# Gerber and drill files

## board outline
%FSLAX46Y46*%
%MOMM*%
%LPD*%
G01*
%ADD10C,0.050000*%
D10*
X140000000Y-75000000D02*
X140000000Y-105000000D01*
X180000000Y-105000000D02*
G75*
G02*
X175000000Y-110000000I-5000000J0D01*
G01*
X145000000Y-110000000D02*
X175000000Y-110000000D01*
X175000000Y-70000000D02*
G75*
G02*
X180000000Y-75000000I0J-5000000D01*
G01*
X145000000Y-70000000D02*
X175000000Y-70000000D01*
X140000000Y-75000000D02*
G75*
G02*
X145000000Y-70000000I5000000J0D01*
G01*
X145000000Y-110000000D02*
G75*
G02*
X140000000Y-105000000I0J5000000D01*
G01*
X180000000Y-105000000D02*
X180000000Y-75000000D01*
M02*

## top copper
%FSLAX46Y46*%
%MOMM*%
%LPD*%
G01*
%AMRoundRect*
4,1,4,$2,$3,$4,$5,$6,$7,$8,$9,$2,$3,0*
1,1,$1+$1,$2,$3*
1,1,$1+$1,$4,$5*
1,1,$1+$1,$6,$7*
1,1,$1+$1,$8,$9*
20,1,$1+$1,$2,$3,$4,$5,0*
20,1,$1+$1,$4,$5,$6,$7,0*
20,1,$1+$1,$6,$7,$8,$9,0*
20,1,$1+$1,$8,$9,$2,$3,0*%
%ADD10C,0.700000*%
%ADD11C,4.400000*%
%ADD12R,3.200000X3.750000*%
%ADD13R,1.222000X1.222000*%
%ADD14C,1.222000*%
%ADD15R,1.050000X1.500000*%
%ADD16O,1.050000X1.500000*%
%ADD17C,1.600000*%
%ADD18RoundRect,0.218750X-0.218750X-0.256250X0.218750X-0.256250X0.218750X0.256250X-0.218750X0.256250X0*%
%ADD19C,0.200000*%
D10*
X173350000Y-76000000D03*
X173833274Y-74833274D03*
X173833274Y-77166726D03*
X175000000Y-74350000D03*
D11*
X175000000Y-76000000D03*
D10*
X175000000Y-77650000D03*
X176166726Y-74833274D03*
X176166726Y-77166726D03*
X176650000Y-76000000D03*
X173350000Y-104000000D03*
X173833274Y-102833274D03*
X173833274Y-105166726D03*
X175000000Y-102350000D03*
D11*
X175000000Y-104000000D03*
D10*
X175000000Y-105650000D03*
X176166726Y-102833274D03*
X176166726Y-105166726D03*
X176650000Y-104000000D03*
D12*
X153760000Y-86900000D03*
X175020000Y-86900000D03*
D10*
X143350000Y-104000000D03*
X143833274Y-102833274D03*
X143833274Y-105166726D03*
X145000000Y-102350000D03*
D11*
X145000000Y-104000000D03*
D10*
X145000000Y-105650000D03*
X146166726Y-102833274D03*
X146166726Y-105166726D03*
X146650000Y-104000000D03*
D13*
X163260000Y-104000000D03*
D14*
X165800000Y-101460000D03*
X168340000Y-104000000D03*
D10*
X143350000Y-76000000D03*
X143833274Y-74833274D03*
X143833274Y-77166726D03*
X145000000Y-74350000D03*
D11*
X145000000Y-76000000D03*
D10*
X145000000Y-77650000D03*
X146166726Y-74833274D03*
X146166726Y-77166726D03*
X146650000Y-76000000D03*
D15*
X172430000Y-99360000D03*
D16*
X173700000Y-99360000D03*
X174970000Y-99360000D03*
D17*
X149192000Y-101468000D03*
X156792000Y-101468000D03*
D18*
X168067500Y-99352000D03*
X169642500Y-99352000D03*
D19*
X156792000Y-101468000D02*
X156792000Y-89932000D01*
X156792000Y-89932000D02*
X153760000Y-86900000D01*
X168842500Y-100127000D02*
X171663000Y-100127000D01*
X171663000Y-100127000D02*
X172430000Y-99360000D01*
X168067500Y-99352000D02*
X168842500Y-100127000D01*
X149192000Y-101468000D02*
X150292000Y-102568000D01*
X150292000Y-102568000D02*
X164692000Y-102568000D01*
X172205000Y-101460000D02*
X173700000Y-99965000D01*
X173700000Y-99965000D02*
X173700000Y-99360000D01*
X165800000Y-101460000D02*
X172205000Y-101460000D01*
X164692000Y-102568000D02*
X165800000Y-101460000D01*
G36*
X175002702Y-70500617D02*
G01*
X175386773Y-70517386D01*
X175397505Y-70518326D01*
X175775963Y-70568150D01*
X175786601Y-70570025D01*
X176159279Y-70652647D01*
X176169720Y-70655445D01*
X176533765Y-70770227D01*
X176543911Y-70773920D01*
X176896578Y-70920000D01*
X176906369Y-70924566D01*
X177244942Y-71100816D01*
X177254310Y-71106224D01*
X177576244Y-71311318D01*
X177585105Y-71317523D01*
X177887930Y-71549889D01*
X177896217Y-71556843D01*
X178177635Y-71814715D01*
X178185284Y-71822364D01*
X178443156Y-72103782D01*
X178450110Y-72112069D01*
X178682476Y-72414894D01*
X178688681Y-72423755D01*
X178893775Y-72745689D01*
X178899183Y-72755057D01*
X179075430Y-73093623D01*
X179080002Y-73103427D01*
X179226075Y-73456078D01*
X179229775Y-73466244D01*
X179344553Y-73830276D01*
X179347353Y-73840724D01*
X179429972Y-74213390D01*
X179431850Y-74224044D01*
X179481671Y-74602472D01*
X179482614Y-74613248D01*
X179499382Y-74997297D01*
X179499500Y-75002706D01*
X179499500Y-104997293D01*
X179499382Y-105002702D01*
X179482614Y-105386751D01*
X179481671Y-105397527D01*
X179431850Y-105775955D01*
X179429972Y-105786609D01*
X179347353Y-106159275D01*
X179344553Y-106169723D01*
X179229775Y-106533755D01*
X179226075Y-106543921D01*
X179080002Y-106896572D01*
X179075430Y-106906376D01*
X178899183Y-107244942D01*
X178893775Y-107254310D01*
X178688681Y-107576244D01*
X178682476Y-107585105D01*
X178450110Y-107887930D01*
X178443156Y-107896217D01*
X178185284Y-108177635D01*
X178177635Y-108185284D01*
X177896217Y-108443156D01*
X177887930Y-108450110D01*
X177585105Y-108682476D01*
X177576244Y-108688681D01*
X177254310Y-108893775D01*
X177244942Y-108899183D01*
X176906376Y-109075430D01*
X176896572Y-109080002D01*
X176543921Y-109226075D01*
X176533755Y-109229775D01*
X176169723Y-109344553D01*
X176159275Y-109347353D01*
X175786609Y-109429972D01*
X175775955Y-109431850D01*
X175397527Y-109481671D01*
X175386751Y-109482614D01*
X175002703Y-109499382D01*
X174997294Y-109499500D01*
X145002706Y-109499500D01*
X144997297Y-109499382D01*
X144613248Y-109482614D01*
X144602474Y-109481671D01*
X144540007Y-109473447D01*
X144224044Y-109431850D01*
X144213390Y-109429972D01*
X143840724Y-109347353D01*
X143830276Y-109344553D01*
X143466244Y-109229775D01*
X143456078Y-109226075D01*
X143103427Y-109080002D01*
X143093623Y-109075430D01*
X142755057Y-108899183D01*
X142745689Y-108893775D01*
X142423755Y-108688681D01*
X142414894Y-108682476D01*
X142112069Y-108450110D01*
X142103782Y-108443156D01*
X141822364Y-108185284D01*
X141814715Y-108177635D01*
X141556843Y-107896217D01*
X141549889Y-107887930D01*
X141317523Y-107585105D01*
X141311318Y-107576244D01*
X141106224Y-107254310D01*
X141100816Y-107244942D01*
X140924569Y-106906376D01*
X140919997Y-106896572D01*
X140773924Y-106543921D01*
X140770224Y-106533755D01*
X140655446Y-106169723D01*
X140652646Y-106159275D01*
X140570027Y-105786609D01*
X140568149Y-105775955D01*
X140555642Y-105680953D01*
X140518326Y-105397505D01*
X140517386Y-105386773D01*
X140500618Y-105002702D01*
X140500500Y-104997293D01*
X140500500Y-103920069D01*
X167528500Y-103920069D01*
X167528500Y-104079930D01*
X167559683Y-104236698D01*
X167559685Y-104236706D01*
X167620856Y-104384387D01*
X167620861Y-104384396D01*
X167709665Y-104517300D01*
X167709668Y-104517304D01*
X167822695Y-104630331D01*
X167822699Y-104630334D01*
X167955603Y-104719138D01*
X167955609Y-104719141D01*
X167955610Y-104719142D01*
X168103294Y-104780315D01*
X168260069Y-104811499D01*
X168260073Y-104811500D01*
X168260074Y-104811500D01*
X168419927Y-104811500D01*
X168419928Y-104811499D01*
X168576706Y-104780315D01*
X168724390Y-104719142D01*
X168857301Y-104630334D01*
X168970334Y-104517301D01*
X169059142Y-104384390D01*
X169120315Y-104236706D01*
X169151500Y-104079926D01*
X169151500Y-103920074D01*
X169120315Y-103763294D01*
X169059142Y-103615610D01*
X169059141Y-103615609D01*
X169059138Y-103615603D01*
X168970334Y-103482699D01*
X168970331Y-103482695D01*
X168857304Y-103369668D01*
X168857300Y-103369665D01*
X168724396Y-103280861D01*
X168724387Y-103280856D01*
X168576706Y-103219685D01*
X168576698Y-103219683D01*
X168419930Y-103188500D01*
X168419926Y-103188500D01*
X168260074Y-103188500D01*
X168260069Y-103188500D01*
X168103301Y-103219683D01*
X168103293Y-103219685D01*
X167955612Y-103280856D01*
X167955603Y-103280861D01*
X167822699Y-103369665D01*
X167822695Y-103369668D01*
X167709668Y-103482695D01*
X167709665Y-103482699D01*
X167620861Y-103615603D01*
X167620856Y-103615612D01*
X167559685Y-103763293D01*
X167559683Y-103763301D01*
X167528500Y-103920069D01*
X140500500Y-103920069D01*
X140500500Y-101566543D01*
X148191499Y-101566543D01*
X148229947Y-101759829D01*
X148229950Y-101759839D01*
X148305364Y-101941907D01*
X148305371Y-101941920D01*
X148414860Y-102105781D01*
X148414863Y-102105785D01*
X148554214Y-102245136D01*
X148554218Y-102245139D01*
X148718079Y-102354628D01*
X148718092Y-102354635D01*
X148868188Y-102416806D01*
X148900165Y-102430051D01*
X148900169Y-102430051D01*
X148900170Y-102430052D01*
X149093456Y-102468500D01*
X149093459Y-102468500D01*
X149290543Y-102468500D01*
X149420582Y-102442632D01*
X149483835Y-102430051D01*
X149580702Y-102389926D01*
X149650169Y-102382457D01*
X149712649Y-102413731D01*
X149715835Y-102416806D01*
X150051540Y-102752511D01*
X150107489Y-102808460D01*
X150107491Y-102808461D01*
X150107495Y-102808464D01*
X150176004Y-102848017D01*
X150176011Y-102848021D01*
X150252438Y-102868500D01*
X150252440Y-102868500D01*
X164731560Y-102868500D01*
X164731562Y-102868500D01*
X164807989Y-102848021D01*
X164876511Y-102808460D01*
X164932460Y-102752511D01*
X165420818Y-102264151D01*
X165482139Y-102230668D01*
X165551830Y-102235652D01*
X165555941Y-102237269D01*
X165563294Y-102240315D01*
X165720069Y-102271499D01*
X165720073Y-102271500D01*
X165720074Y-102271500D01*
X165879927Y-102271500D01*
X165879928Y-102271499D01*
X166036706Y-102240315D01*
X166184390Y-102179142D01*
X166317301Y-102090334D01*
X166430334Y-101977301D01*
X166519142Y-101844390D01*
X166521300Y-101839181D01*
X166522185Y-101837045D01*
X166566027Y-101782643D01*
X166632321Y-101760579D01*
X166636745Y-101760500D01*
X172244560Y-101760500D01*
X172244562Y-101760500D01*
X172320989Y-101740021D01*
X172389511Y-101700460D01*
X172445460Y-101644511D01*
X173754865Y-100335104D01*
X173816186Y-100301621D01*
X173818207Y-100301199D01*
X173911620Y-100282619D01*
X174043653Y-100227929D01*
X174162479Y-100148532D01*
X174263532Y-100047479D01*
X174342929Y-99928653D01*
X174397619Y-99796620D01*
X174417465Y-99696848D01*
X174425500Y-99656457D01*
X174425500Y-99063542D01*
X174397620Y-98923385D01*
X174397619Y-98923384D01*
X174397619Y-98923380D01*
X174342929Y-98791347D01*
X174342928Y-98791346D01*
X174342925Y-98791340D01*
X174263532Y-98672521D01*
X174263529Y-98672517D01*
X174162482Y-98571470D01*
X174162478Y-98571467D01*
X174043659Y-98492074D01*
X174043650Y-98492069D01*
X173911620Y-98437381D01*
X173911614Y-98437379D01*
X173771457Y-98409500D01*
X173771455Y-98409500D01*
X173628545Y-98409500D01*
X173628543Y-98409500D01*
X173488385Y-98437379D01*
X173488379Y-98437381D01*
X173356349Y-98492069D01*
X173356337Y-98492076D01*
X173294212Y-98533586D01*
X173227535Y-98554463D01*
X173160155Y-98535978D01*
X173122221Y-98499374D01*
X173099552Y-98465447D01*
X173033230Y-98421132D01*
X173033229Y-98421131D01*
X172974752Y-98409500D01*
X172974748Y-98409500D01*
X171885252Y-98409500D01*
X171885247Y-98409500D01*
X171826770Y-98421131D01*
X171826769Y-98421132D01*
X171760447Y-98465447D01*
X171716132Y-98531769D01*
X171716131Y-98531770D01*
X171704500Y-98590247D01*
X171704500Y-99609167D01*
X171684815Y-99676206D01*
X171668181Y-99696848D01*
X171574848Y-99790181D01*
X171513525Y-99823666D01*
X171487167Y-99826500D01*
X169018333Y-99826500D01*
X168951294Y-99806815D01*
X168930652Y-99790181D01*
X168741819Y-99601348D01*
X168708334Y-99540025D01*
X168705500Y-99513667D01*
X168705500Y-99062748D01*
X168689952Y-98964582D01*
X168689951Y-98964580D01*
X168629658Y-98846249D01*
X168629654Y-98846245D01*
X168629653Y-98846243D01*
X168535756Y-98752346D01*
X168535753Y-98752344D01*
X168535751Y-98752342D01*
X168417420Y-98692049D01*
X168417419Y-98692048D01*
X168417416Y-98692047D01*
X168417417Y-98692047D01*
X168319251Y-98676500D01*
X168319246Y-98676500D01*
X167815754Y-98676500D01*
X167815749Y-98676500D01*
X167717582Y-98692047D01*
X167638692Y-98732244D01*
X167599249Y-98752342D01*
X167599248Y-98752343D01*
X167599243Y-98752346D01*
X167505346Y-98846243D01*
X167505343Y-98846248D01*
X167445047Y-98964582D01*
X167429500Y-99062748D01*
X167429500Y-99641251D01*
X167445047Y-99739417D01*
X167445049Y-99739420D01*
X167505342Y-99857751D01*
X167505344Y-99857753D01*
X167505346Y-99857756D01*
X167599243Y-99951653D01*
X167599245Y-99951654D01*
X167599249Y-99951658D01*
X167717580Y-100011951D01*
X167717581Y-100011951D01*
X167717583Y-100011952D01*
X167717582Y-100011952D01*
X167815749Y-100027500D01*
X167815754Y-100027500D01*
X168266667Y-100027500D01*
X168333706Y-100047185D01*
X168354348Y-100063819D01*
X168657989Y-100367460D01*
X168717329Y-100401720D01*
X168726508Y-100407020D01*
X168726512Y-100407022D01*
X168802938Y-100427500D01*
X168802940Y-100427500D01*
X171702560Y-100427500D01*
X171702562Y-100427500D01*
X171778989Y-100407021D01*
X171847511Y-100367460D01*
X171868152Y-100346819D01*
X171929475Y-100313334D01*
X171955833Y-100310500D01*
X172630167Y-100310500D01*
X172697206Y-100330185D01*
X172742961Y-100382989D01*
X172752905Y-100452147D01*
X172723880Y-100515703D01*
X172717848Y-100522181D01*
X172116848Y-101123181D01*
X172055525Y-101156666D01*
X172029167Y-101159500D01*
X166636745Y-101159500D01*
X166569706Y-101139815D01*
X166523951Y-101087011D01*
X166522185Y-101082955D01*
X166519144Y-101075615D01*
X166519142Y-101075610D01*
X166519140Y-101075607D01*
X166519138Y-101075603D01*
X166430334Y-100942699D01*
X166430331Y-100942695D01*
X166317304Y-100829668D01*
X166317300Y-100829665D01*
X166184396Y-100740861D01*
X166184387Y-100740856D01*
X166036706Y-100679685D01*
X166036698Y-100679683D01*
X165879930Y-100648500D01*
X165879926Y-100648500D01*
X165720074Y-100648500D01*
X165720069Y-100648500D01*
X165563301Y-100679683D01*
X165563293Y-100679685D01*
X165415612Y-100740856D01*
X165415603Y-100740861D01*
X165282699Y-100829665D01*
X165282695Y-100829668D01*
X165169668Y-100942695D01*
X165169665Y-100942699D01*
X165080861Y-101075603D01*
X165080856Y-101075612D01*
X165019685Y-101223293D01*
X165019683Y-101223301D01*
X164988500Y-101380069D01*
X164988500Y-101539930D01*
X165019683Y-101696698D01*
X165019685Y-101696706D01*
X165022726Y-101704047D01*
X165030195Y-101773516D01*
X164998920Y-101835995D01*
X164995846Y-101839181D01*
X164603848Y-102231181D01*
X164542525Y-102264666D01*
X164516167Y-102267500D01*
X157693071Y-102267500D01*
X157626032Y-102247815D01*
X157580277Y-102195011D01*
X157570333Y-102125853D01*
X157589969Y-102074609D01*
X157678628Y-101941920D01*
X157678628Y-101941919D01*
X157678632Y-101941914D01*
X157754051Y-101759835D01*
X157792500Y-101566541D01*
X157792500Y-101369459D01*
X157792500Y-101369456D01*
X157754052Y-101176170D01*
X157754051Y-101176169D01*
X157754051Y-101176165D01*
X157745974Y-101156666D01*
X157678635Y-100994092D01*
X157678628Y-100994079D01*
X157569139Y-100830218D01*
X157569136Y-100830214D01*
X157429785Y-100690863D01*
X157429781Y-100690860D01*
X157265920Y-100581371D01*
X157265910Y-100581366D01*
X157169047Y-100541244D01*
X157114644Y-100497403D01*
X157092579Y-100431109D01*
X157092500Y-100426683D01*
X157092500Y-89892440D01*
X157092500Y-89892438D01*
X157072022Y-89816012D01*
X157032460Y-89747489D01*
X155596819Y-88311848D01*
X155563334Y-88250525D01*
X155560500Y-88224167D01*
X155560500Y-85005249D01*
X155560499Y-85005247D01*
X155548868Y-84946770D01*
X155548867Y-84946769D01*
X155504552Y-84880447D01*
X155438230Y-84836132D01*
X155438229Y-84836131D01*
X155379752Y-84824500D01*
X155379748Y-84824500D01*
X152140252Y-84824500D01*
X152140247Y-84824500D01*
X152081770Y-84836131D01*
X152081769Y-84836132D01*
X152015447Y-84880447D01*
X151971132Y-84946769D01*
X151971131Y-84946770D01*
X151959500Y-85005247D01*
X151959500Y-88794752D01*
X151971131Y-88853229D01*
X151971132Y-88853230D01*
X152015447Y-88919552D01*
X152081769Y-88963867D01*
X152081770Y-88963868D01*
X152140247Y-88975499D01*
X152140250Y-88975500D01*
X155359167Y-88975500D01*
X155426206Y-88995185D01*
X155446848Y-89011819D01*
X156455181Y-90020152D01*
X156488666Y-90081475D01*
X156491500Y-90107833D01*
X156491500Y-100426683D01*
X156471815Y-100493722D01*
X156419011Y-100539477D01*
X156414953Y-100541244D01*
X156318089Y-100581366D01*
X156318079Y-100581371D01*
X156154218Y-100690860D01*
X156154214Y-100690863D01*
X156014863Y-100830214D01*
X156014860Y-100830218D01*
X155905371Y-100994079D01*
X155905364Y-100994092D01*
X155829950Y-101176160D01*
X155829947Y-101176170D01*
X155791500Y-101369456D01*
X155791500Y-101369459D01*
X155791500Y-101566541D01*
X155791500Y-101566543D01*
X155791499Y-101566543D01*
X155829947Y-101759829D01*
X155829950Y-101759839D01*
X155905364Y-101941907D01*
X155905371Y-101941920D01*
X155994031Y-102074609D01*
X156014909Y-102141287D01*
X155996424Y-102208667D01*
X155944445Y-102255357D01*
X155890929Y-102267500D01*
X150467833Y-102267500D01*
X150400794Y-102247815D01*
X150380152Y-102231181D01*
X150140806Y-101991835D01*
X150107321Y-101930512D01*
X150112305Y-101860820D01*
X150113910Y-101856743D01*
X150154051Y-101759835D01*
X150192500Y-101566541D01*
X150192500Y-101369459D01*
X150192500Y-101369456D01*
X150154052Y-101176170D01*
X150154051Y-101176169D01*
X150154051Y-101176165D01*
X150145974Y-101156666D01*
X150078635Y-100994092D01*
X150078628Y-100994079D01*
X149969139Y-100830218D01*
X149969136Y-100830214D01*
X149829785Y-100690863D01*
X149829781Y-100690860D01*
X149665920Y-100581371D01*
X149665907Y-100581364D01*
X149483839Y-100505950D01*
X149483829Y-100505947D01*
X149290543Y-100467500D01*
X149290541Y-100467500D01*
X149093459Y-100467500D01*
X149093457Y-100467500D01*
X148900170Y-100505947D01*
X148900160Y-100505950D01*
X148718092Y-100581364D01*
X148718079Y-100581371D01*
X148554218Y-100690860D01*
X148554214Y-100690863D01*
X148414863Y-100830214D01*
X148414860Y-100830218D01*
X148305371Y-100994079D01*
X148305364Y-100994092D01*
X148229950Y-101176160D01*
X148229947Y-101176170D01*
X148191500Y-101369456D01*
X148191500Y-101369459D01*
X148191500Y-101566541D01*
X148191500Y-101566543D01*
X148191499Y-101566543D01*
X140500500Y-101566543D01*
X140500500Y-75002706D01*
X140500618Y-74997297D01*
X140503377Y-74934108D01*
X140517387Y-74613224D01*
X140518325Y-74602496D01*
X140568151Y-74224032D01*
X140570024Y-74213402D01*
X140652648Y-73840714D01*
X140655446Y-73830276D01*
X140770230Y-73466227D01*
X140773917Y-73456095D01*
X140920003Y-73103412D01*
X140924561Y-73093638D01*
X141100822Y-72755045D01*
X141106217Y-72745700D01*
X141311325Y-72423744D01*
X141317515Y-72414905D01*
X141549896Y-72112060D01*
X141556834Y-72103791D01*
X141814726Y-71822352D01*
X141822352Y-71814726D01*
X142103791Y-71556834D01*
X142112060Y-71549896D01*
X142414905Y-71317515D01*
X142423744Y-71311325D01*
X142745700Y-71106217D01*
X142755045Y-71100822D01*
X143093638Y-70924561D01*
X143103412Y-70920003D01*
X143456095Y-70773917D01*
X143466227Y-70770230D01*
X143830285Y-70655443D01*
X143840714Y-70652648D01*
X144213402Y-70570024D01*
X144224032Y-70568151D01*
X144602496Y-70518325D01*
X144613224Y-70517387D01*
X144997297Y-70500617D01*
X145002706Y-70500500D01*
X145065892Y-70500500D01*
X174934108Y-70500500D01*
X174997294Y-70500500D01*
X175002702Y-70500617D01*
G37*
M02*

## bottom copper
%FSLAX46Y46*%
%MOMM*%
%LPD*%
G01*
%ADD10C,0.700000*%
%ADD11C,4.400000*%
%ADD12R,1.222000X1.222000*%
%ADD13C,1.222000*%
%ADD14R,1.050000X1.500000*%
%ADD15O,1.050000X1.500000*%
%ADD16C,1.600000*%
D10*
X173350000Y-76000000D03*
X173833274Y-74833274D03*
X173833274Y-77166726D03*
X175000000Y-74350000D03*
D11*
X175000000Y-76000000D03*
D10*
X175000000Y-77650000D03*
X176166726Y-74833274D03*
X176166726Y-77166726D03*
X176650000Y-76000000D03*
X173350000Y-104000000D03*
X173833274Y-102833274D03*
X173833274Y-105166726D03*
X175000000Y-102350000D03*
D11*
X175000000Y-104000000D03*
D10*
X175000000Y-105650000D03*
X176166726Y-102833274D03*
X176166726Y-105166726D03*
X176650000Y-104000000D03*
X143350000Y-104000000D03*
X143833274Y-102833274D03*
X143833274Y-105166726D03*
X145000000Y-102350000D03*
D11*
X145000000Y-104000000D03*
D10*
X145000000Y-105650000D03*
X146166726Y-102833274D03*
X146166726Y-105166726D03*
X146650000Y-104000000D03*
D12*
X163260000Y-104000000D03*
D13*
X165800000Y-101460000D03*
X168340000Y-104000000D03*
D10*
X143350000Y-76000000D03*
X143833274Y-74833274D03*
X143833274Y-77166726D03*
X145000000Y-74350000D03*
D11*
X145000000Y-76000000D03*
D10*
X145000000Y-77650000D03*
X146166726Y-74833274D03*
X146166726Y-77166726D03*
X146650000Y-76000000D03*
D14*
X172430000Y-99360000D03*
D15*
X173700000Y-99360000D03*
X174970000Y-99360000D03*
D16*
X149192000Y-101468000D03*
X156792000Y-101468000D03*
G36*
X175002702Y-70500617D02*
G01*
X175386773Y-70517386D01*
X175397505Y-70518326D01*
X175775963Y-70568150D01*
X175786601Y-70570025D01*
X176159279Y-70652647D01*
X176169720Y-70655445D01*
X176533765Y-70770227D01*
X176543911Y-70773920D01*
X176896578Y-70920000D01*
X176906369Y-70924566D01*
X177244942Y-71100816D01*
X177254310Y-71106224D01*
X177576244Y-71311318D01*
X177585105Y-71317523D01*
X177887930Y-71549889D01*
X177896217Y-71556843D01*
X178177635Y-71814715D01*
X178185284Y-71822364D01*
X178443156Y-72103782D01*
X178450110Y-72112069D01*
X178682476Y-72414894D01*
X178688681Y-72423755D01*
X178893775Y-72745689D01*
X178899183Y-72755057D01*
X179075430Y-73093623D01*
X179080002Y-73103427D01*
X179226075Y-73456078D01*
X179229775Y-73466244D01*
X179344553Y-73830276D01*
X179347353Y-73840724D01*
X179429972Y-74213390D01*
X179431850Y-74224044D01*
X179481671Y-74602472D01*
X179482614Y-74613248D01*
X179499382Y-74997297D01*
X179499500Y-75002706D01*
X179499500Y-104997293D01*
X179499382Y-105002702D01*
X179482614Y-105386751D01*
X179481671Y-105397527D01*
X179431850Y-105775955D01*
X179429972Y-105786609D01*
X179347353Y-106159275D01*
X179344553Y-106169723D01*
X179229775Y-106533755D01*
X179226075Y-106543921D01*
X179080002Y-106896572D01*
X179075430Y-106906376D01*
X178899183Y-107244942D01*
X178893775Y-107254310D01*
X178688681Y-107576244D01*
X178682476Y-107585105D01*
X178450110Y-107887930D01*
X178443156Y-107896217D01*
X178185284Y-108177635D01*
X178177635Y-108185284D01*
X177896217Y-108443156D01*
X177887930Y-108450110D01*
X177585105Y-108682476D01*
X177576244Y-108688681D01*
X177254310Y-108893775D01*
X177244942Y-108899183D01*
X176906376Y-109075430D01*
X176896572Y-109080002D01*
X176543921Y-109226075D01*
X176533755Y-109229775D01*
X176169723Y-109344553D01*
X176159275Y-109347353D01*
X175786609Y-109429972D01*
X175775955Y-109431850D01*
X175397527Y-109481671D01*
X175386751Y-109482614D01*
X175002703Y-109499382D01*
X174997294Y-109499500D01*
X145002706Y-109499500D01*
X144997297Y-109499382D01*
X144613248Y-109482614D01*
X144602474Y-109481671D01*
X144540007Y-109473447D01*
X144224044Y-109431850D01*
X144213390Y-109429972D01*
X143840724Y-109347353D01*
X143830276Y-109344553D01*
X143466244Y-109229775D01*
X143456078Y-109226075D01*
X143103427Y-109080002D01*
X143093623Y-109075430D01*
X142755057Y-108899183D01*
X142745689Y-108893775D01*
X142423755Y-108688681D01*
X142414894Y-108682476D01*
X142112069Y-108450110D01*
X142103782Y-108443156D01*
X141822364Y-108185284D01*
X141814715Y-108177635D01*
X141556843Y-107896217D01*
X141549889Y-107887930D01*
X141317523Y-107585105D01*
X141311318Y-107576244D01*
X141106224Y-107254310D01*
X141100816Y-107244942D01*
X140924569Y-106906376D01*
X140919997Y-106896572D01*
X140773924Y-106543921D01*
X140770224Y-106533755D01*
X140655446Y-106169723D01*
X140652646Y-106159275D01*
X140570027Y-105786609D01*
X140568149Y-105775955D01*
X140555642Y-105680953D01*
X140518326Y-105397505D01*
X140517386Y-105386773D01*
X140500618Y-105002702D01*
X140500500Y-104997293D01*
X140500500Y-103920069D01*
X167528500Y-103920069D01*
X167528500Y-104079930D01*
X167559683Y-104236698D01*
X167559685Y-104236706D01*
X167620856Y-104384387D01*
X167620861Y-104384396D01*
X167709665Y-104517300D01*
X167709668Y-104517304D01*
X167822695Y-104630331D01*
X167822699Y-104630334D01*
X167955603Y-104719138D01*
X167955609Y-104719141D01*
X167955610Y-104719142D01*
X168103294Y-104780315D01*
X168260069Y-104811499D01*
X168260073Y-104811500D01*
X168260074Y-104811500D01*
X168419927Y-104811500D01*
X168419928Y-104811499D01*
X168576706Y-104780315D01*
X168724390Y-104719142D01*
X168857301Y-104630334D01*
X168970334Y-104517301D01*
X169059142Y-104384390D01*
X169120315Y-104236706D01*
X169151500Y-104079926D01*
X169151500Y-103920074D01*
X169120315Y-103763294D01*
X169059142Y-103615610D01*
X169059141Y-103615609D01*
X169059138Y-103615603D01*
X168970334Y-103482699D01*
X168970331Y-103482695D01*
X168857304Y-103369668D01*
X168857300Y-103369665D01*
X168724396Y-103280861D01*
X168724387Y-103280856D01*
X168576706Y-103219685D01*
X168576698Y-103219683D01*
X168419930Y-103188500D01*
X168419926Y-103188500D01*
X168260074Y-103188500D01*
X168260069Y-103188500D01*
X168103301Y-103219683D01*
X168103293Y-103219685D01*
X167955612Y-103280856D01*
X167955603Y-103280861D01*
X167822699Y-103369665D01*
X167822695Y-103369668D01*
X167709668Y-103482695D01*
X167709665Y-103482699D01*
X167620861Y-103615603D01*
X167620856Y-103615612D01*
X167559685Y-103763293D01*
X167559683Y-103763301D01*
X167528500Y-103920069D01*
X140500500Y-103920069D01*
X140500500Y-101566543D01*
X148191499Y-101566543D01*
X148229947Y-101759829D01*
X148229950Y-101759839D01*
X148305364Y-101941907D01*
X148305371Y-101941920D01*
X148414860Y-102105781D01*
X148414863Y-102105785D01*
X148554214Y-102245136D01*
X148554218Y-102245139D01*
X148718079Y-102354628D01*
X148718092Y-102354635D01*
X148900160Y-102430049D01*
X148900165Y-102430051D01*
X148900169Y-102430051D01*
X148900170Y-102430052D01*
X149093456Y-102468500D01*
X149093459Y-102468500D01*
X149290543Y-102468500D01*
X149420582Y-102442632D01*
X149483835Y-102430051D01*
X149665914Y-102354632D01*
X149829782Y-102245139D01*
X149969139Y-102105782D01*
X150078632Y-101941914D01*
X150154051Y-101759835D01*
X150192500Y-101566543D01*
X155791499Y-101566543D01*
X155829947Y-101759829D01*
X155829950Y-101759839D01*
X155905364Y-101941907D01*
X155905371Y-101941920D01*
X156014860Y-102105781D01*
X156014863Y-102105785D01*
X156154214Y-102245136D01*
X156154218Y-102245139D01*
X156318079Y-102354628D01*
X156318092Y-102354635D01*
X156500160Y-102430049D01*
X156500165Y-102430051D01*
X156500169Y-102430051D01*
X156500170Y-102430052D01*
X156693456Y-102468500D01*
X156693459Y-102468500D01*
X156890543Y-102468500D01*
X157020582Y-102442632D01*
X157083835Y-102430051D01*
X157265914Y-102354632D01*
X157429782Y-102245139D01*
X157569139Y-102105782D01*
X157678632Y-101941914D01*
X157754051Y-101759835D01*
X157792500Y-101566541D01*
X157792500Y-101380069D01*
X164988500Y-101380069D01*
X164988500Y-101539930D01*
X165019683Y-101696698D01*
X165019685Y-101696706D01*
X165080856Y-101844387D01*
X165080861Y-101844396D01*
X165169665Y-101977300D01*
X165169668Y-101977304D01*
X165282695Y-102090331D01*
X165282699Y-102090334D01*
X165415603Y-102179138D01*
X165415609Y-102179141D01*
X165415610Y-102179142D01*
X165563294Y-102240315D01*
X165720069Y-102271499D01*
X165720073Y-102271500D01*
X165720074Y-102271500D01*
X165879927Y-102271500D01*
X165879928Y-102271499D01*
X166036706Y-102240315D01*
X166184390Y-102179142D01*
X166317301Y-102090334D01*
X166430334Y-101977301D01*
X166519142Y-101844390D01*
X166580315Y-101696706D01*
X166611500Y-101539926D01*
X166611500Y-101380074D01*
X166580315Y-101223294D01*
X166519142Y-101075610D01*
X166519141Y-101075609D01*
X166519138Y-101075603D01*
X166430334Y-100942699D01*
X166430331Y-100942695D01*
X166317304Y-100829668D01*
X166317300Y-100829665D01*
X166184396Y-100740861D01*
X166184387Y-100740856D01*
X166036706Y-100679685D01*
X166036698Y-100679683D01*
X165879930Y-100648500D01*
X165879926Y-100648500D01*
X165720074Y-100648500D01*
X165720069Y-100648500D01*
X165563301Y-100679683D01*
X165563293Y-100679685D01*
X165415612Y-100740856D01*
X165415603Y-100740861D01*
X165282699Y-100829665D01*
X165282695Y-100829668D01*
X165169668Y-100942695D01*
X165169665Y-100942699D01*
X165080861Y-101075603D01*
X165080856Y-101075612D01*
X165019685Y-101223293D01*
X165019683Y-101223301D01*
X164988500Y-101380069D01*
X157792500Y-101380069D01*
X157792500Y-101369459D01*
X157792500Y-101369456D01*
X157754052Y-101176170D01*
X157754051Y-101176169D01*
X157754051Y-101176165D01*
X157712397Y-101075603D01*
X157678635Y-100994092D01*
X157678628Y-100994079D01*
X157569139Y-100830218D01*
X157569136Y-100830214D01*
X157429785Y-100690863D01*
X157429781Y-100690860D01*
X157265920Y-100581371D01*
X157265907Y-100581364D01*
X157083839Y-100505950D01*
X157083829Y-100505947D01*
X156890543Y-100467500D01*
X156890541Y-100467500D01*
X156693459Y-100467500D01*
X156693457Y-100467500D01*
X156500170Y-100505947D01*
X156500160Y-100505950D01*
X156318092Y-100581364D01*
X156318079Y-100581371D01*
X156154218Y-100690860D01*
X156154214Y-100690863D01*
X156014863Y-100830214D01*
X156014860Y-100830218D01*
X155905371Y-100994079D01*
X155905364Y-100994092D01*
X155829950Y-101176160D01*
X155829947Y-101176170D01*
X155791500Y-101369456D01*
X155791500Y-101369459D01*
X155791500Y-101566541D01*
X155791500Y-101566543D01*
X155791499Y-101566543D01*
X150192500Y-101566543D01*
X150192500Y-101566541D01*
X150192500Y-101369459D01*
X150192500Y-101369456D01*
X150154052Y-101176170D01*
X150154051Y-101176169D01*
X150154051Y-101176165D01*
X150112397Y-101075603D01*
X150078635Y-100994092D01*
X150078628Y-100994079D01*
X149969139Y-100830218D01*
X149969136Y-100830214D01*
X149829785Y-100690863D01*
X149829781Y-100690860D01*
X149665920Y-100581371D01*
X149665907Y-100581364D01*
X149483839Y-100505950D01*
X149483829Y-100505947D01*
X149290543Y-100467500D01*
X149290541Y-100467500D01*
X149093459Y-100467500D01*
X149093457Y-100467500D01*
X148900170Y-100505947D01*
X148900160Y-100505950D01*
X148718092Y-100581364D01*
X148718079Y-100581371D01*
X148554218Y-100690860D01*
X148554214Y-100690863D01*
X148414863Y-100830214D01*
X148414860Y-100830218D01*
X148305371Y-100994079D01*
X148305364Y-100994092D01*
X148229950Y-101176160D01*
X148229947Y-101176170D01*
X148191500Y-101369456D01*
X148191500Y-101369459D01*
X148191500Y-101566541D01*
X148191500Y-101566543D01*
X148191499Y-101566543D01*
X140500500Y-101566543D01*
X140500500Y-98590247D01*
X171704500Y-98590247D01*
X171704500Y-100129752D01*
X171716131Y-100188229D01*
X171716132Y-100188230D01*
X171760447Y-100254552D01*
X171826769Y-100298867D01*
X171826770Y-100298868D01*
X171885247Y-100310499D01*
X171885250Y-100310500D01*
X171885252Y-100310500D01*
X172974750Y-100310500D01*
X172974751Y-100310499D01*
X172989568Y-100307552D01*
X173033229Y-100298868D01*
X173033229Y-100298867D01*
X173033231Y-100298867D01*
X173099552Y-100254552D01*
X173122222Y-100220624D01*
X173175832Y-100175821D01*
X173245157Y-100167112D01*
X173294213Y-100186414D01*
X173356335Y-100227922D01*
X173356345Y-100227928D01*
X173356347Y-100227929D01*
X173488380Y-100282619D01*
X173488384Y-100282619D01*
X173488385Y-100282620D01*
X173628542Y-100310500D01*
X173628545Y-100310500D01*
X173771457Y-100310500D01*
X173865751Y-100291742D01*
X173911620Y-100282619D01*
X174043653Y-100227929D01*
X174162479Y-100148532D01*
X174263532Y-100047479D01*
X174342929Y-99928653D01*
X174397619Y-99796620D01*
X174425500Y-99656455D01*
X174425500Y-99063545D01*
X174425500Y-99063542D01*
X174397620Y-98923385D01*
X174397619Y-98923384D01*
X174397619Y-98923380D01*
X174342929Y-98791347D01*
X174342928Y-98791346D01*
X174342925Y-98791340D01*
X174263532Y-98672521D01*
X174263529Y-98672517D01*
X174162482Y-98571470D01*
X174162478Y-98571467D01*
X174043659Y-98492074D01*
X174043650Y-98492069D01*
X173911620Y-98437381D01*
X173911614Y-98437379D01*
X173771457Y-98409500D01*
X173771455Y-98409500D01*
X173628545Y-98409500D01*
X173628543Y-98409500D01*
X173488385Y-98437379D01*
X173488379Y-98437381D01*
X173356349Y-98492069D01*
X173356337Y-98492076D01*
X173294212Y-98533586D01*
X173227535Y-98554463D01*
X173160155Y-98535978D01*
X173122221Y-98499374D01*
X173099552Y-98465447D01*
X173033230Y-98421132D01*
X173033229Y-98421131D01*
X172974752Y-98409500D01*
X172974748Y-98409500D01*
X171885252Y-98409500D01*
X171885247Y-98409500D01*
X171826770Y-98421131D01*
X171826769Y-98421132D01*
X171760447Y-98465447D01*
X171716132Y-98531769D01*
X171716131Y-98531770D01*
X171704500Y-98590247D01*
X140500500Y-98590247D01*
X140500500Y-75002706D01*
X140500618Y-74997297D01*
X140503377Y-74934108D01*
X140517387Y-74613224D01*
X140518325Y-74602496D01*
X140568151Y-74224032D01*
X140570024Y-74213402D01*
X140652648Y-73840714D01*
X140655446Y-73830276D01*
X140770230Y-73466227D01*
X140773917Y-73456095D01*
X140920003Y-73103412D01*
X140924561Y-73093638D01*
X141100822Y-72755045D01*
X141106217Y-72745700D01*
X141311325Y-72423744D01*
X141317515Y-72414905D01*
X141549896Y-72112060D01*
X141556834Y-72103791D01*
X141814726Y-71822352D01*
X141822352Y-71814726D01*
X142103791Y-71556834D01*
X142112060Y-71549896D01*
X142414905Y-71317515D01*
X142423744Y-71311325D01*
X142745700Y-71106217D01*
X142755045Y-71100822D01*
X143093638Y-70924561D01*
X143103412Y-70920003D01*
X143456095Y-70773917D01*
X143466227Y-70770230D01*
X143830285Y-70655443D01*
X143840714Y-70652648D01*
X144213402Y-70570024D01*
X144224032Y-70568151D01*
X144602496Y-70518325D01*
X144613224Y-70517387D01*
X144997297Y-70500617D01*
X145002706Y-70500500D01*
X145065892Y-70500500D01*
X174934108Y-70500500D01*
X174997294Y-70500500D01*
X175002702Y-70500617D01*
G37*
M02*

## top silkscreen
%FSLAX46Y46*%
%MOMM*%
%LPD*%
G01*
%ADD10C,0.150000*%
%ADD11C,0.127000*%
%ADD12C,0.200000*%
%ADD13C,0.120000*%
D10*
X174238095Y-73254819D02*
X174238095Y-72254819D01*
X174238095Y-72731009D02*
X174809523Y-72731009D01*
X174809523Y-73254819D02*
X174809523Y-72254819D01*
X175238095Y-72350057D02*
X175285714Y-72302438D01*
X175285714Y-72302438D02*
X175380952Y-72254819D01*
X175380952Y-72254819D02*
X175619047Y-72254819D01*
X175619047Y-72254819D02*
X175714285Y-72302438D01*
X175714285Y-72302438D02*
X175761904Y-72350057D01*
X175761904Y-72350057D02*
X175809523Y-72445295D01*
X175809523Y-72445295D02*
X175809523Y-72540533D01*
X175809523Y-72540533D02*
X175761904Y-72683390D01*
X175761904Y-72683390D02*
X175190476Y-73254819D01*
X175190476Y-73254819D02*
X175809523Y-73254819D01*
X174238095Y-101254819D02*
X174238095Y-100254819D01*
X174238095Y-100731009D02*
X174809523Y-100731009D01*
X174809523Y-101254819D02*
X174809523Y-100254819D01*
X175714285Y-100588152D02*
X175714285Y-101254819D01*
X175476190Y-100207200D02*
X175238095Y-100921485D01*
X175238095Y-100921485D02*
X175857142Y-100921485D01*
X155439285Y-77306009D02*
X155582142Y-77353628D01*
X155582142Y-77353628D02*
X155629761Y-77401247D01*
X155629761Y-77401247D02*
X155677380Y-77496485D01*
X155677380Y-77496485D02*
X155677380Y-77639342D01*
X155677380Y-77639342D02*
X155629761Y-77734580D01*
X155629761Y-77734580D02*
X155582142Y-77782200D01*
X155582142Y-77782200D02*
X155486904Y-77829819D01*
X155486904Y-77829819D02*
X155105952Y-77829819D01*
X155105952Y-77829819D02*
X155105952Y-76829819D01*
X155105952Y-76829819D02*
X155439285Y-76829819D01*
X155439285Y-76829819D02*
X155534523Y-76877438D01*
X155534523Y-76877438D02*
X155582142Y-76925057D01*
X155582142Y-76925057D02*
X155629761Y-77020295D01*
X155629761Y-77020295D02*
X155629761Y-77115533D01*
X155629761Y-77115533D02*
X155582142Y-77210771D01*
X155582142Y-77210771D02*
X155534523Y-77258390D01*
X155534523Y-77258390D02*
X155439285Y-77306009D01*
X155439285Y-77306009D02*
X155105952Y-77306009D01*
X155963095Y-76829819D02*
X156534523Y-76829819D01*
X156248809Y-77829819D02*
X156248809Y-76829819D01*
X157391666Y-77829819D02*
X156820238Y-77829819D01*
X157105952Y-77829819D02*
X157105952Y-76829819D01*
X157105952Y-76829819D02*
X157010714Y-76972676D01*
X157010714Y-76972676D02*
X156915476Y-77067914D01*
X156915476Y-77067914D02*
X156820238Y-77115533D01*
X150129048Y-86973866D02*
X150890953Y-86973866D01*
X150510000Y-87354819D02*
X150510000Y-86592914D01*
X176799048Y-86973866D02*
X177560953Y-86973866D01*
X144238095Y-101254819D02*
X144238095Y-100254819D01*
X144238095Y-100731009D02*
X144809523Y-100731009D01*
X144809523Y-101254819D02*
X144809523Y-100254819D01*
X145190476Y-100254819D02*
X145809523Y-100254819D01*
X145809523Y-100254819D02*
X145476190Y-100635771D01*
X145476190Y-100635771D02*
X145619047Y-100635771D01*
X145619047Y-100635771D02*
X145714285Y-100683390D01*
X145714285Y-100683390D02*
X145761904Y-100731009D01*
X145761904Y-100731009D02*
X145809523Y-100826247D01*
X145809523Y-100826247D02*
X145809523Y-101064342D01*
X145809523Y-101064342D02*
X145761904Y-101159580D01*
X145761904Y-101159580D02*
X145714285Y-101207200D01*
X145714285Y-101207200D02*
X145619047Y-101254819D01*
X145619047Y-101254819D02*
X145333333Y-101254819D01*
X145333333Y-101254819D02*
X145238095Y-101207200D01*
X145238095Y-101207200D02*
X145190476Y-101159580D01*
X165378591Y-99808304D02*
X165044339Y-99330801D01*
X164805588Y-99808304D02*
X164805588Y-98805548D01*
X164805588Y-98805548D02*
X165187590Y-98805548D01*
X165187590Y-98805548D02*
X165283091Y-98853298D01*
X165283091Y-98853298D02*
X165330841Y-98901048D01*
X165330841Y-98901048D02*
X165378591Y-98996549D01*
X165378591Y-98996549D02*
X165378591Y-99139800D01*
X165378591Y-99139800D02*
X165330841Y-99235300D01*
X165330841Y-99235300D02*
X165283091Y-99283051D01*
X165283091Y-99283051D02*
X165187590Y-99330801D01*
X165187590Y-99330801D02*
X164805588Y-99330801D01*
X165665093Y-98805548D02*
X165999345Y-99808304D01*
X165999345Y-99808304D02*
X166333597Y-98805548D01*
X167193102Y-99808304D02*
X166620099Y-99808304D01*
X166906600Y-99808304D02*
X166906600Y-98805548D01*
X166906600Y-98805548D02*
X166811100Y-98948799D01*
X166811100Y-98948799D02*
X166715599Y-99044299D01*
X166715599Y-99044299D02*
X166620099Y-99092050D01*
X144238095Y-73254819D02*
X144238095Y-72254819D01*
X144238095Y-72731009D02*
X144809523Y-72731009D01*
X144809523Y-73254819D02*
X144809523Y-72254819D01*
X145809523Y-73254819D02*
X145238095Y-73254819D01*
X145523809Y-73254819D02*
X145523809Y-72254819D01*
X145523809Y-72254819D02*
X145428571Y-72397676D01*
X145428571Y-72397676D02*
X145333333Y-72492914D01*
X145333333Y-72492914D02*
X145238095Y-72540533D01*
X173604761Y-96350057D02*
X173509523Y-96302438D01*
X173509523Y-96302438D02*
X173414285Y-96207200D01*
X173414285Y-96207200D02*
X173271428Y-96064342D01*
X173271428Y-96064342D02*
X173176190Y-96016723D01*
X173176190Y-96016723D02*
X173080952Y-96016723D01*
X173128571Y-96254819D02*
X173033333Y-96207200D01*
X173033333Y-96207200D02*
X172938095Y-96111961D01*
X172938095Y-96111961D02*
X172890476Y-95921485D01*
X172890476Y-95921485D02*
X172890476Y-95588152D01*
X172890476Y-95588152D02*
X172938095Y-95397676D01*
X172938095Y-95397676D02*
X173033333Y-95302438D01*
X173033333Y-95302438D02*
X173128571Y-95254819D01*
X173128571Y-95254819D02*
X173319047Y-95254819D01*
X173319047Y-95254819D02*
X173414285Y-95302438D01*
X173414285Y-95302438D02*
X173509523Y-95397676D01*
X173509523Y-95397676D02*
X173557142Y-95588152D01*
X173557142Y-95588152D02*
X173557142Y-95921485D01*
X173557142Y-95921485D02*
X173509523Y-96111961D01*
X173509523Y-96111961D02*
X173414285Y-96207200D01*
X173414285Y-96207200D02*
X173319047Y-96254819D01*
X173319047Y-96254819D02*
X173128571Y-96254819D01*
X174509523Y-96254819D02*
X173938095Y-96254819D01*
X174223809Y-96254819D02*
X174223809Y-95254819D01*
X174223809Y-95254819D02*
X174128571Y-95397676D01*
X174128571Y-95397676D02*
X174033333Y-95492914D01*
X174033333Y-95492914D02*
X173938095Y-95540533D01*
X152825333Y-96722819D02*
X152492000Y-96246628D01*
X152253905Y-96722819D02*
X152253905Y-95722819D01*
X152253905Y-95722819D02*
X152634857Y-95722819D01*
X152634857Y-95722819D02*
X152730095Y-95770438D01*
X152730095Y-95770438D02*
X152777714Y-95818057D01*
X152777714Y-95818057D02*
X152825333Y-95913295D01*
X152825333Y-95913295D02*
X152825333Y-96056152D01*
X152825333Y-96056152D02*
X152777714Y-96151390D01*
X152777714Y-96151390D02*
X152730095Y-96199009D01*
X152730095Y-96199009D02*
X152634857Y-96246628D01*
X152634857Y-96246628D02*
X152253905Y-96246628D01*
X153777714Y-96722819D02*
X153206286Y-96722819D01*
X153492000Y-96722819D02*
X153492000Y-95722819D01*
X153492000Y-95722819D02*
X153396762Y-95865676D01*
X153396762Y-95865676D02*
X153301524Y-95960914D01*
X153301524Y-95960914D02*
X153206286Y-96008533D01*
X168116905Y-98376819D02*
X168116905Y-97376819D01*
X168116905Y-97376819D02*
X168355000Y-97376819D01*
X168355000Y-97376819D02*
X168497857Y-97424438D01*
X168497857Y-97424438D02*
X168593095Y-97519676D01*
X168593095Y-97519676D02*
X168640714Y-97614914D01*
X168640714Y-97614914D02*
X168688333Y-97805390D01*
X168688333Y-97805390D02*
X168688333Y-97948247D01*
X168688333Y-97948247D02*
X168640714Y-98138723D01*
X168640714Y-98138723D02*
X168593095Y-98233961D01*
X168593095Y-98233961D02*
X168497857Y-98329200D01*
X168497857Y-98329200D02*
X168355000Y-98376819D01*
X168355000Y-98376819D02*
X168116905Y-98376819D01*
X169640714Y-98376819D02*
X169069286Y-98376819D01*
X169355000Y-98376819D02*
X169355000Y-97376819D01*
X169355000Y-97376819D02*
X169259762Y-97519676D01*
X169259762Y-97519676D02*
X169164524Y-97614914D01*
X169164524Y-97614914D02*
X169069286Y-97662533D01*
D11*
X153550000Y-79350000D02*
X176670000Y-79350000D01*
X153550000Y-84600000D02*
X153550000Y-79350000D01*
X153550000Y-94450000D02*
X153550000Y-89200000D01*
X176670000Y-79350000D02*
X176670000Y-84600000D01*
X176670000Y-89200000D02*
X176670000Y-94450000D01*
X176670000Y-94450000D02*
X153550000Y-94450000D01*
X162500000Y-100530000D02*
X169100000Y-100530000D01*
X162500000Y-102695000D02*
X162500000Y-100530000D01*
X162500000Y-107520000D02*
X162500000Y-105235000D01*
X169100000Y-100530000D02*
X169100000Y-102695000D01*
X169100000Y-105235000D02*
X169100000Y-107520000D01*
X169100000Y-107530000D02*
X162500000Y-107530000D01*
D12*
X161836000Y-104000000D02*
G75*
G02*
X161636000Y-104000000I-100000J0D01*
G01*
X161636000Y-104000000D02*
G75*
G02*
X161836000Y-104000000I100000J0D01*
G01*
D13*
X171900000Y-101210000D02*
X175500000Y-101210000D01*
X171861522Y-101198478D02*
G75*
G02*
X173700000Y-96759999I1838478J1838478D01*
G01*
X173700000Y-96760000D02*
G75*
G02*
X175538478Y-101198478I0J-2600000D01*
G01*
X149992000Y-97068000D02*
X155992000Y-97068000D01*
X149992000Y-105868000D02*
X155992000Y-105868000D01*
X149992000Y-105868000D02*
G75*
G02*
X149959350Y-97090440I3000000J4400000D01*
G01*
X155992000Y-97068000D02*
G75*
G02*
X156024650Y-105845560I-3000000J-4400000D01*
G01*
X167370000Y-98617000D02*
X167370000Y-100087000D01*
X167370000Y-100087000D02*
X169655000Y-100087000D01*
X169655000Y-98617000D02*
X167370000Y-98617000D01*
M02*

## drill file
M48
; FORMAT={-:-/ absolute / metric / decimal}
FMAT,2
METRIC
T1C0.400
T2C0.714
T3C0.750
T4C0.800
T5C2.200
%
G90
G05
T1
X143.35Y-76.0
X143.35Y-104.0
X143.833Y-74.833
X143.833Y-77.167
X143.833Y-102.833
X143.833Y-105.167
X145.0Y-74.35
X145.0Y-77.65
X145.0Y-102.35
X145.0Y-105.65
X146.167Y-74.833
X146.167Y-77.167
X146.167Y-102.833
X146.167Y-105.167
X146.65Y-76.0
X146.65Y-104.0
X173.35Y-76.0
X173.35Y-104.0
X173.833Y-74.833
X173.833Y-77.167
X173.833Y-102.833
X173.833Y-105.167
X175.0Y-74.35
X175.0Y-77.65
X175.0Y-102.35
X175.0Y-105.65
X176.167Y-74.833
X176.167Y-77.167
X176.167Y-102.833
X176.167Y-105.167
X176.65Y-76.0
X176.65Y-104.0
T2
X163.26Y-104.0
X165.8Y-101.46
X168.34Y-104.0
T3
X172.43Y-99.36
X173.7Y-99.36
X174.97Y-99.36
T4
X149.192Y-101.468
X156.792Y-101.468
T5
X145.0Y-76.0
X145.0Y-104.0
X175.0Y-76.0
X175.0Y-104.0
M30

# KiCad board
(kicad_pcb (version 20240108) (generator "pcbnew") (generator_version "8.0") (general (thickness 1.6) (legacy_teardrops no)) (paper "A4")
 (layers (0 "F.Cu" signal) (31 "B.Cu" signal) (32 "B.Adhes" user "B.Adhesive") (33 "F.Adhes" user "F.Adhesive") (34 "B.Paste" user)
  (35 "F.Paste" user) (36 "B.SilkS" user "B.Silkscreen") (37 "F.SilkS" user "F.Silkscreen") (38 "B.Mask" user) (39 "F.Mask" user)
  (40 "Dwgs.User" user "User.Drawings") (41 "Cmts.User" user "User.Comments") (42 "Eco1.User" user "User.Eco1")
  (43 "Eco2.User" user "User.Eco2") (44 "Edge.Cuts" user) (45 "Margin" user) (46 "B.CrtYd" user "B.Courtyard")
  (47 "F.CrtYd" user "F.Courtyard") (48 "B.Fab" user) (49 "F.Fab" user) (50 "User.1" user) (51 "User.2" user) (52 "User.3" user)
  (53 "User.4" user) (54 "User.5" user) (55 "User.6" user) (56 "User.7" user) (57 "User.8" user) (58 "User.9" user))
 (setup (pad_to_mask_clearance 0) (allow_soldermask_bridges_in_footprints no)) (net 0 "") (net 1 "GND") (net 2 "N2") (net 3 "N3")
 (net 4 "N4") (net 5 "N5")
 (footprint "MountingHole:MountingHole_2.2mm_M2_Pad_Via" (layer "F.Cu") (at 175 76)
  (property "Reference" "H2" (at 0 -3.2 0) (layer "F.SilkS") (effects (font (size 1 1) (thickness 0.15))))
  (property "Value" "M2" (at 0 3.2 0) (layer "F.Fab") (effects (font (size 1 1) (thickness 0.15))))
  (pad "1" thru_hole circle (at -1.65 0) (size 0.7 0.7) (drill 0.4) (layers "*.Cu" "*.Mask") (remove_unused_layers no) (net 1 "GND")
   (zone_connect 2))
  (pad "1" thru_hole circle (at -1.166726 -1.166726) (size 0.7 0.7) (drill 0.4) (layers "*.Cu" "*.Mask") (remove_unused_layers no)
   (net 1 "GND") (zone_connect 2))
  (pad "1" thru_hole circle (at -1.166726 1.166726) (size 0.7 0.7) (drill 0.4) (layers "*.Cu" "*.Mask") (remove_unused_layers no)
   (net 1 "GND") (zone_connect 2))
  (pad "1" thru_hole circle (at 0 -1.65) (size 0.7 0.7) (drill 0.4) (layers "*.Cu" "*.Mask") (remove_unused_layers no) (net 1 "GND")
   (zone_connect 2))
  (pad "1" thru_hole circle (at 0 0) (size 4.4 4.4) (drill 2.2) (layers "*.Cu" "*.Mask") (remove_unused_layers no) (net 1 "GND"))
  (pad "1" thru_hole circle (at 0 1.65) (size 0.7 0.7) (drill 0.4) (layers "*.Cu" "*.Mask") (remove_unused_layers no) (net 1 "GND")
   (zone_connect 2))
  (pad "1" thru_hole circle (at 1.166726 -1.166726) (size 0.7 0.7) (drill 0.4) (layers "*.Cu" "*.Mask") (remove_unused_layers no)
   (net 1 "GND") (zone_connect 2))
  (pad "1" thru_hole circle (at 1.166726 1.166726) (size 0.7 0.7) (drill 0.4) (layers "*.Cu" "*.Mask") (remove_unused_layers no)
   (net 1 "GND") (zone_connect 2))
  (pad "1" thru_hole circle (at 1.65 0) (size 0.7 0.7) (drill 0.4) (layers "*.Cu" "*.Mask") (remove_unused_layers no) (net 1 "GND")
   (zone_connect 2)))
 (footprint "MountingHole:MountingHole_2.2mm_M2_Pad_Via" (layer "F.Cu") (at 175 104)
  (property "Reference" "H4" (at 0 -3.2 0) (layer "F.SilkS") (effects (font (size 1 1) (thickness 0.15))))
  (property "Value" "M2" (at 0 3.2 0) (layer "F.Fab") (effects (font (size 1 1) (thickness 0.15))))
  (pad "1" thru_hole circle (at -1.65 0) (size 0.7 0.7) (drill 0.4) (layers "*.Cu" "*.Mask") (remove_unused_layers no) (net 1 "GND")
   (zone_connect 2))
  (pad "1" thru_hole circle (at -1.166726 -1.166726) (size 0.7 0.7) (drill 0.4) (layers "*.Cu" "*.Mask") (remove_unused_layers no)
   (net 1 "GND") (zone_connect 2))
  (pad "1" thru_hole circle (at -1.166726 1.166726) (size 0.7 0.7) (drill 0.4) (layers "*.Cu" "*.Mask") (remove_unused_layers no)
   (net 1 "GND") (zone_connect 2))
  (pad "1" thru_hole circle (at 0 -1.65) (size 0.7 0.7) (drill 0.4) (layers "*.Cu" "*.Mask") (remove_unused_layers no) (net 1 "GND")
   (zone_connect 2))
  (pad "1" thru_hole circle (at 0 0) (size 4.4 4.4) (drill 2.2) (layers "*.Cu" "*.Mask") (remove_unused_layers no) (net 1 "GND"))
  (pad "1" thru_hole circle (at 0 1.65) (size 0.7 0.7) (drill 0.4) (layers "*.Cu" "*.Mask") (remove_unused_layers no) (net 1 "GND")
   (zone_connect 2))
  (pad "1" thru_hole circle (at 1.166726 -1.166726) (size 0.7 0.7) (drill 0.4) (layers "*.Cu" "*.Mask") (remove_unused_layers no)
   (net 1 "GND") (zone_connect 2))
  (pad "1" thru_hole circle (at 1.166726 1.166726) (size 0.7 0.7) (drill 0.4) (layers "*.Cu" "*.Mask") (remove_unused_layers no)
   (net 1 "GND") (zone_connect 2))
  (pad "1" thru_hole circle (at 1.65 0) (size 0.7 0.7) (drill 0.4) (layers "*.Cu" "*.Mask") (remove_unused_layers no) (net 1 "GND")
   (zone_connect 2)))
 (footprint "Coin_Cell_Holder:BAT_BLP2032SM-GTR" (layer "F.Cu") (at 165.75 86.9)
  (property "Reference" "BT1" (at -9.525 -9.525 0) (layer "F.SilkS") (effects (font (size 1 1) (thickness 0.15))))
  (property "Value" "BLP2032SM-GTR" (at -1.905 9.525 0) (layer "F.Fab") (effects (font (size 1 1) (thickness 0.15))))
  (fp_line (start -12.2 -7.55) (end 10.92 -7.55) (stroke (width 0.127) (type solid)) (layer "F.SilkS"))
  (fp_line (start -12.2 -2.3) (end -12.2 -7.55) (stroke (width 0.127) (type solid)) (layer "F.SilkS"))
  (fp_line (start -12.2 7.55) (end -12.2 2.3) (stroke (width 0.127) (type solid)) (layer "F.SilkS"))
  (fp_line (start 10.92 -7.55) (end 10.92 -2.3) (stroke (width 0.127) (type solid)) (layer "F.SilkS"))
  (fp_line (start 10.92 2.3) (end 10.92 7.55) (stroke (width 0.127) (type solid)) (layer "F.SilkS"))
  (fp_line (start 10.92 7.55) (end -12.2 7.55) (stroke (width 0.127) (type solid)) (layer "F.SilkS"))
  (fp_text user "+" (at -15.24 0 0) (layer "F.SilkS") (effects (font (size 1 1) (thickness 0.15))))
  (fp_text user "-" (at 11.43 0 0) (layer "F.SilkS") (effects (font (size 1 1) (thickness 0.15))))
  (pad "+" smd rect (at -11.99 0) (size 3.2 3.75) (layers "F.Cu" "F.Paste" "F.Mask") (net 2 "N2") (solder_mask_margin 0.102))
  (pad "-" smd rect (at 9.27 0) (size 3.2 3.75) (layers "F.Cu" "F.Paste" "F.Mask") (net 1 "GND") (solder_mask_margin 0.102)))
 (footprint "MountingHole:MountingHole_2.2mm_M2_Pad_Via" (layer "F.Cu") (at 145 104)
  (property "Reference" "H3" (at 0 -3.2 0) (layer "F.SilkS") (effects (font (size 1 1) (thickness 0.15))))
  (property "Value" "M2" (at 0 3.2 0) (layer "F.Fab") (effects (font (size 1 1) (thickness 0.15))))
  (pad "1" thru_hole circle (at -1.65 0) (size 0.7 0.7) (drill 0.4) (layers "*.Cu" "*.Mask") (remove_unused_layers no) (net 1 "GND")
   (zone_connect 2))
  (pad "1" thru_hole circle (at -1.166726 -1.166726) (size 0.7 0.7) (drill 0.4) (layers "*.Cu" "*.Mask") (remove_unused_layers no)
   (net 1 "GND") (zone_connect 2))
  (pad "1" thru_hole circle (at -1.166726 1.166726) (size 0.7 0.7) (drill 0.4) (layers "*.Cu" "*.Mask") (remove_unused_layers no)
   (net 1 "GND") (zone_connect 2))
  (pad "1" thru_hole circle (at 0 -1.65) (size 0.7 0.7) (drill 0.4) (layers "*.Cu" "*.Mask") (remove_unused_layers no) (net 1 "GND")
   (zone_connect 2))
  (pad "1" thru_hole circle (at 0 0) (size 4.4 4.4) (drill 2.2) (layers "*.Cu" "*.Mask") (remove_unused_layers no) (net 1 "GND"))
  (pad "1" thru_hole circle (at 0 1.65) (size 0.7 0.7) (drill 0.4) (layers "*.Cu" "*.Mask") (remove_unused_layers no) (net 1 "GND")
   (zone_connect 2))
  (pad "1" thru_hole circle (at 1.166726 -1.166726) (size 0.7 0.7) (drill 0.4) (layers "*.Cu" "*.Mask") (remove_unused_layers no)
   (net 1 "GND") (zone_connect 2))
  (pad "1" thru_hole circle (at 1.166726 1.166726) (size 0.7 0.7) (drill 0.4) (layers "*.Cu" "*.Mask") (remove_unused_layers no)
   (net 1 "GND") (zone_connect 2))
  (pad "1" thru_hole circle (at 1.65 0) (size 0.7 0.7) (drill 0.4) (layers "*.Cu" "*.Mask") (remove_unused_layers no) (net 1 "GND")
   (zone_connect 2)))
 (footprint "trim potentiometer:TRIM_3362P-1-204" (layer "F.Cu") (at 165.8 104)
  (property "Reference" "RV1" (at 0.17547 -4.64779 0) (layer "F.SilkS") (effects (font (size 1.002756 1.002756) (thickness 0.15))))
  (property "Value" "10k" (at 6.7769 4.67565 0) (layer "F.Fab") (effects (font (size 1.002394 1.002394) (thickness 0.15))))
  (fp_line (start -3.3 -3.47) (end 3.3 -3.47) (stroke (width 0.127) (type solid)) (layer "F.SilkS"))
  (fp_line (start -3.3 -1.305) (end -3.3 -3.47) (stroke (width 0.127) (type solid)) (layer "F.SilkS"))
  (fp_line (start -3.3 3.52) (end -3.3 1.235) (stroke (width 0.127) (type solid)) (layer "F.SilkS"))
  (fp_line (start 3.3 -3.47) (end 3.3 -1.305) (stroke (width 0.127) (type solid)) (layer "F.SilkS"))
  (fp_line (start 3.3 1.235) (end 3.3 3.52) (stroke (width 0.127) (type solid)) (layer "F.SilkS"))
  (fp_line (start 3.3 3.53) (end -3.3 3.53) (stroke (width 0.127) (type solid)) (layer "F.SilkS"))
  (fp_circle (center -4.064 0) (end -3.964 0) (stroke (width 0.2) (type solid)) (fill none) (layer "F.SilkS"))
  (pad "1" thru_hole rect (at -2.54 0) (size 1.222 1.222) (drill 0.714) (layers "*.Cu" "*.Mask") (remove_unused_layers no) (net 1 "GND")
   (solder_mask_margin 0.102))
  (pad "2" thru_hole circle (at 0 -2.54) (size 1.222 1.222) (drill 0.714) (layers "*.Cu" "*.Mask") (remove_unused_layers no) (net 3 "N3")
   (solder_mask_margin 0.102))
  (pad "3" thru_hole circle (at 2.54 0) (size 1.222 1.222) (drill 0.714) (layers "*.Cu" "*.Mask") (remove_unused_layers no) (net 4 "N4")
   (solder_mask_margin 0.102)))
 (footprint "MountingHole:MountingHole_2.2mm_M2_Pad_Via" (layer "F.Cu") (at 145 76)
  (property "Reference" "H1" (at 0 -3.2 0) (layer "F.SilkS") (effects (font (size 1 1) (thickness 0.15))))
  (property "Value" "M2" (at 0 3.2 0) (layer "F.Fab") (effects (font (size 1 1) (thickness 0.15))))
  (pad "1" thru_hole circle (at -1.65 0) (size 0.7 0.7) (drill 0.4) (layers "*.Cu" "*.Mask") (remove_unused_layers no) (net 1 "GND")
   (zone_connect 2))
  (pad "1" thru_hole circle (at -1.166726 -1.166726) (size 0.7 0.7) (drill 0.4) (layers "*.Cu" "*.Mask") (remove_unused_layers no)
   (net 1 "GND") (zone_connect 2))
  (pad "1" thru_hole circle (at -1.166726 1.166726) (size 0.7 0.7) (drill 0.4) (layers "*.Cu" "*.Mask") (remove_unused_layers no)
   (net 1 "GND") (zone_connect 2))
  (pad "1" thru_hole circle (at 0 -1.65) (size 0.7 0.7) (drill 0.4) (layers "*.Cu" "*.Mask") (remove_unused_layers no) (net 1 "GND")
   (zone_connect 2))
  (pad "1" thru_hole circle (at 0 0) (size 4.4 4.4) (drill 2.2) (layers "*.Cu" "*.Mask") (remove_unused_layers no) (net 1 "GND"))
  (pad "1" thru_hole circle (at 0 1.65) (size 0.7 0.7) (drill 0.4) (layers "*.Cu" "*.Mask") (remove_unused_layers no) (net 1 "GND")
   (zone_connect 2))
  (pad "1" thru_hole circle (at 1.166726 -1.166726) (size 0.7 0.7) (drill 0.4) (layers "*.Cu" "*.Mask") (remove_unused_layers no)
   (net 1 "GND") (zone_connect 2))
  (pad "1" thru_hole circle (at 1.166726 1.166726) (size 0.7 0.7) (drill 0.4) (layers "*.Cu" "*.Mask") (remove_unused_layers no)
   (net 1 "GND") (zone_connect 2))
  (pad "1" thru_hole circle (at 1.65 0) (size 0.7 0.7) (drill 0.4) (layers "*.Cu" "*.Mask") (remove_unused_layers no) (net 1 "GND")
   (zone_connect 2)))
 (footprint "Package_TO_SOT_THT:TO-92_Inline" (layer "F.Cu") (at 172.43 99.36)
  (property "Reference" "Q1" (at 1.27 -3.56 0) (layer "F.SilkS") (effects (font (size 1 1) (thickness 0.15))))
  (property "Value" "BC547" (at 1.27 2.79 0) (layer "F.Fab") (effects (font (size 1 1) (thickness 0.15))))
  (fp_line (start -0.53 1.85) (end 3.07 1.85) (stroke (width 0.12) (type solid)) (layer "F.SilkS"))
  (fp_arc (start -0.568478 1.838478) (mid -1.132087 -0.994977) (end 1.27 -2.6) (stroke (width 0.12) (type solid)) (layer "F.SilkS"))
  (fp_arc (start 1.27 -2.6) (mid 3.672087 -0.994977) (end 3.108478 1.838478) (stroke (width 0.12) (type solid)) (layer "F.SilkS"))
  (pad "1" thru_hole rect (at 0 0) (size 1.05 1.5) (drill 0.75) (layers "*.Cu" "*.Mask") (remove_unused_layers no) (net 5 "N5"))
  (pad "2" thru_hole oval (at 1.27 0) (size 1.05 1.5) (drill 0.75) (layers "*.Cu" "*.Mask") (remove_unused_layers no) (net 3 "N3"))
  (pad "3" thru_hole oval (at 2.54 0) (size 1.05 1.5) (drill 0.75) (layers "*.Cu" "*.Mask") (remove_unused_layers no) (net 1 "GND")))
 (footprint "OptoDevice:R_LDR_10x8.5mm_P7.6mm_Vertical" (layer "F.Cu") (at 149.192 101.468)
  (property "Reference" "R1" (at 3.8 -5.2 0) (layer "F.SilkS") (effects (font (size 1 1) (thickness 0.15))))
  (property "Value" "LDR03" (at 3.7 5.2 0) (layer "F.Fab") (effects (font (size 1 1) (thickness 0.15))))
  (fp_line (start 0.8 -4.4) (end 6.8 -4.4) (stroke (width 0.12) (type solid)) (layer "F.SilkS"))
  (fp_line (start 0.8 4.4) (end 6.8 4.4) (stroke (width 0.12) (type solid)) (layer "F.SilkS"))
  (fp_arc (start 0.8 4.4) (mid -1.525374 0.019809) (end 0.76735 -4.37756) (stroke (width 0.12) (type solid)) (layer "F.SilkS"))
  (fp_arc (start 6.8 -4.4) (mid 9.125374 -0.019809) (end 6.83265 4.37756) (stroke (width 0.12) (type solid)) (layer "F.SilkS"))
  (pad "1" thru_hole circle (at 0 0) (size 1.6 1.6) (drill 0.8) (layers "*.Cu" "*.Mask") (remove_unused_layers no) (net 3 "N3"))
  (pad "2" thru_hole circle (at 7.6 0) (size 1.6 1.6) (drill 0.8) (layers "*.Cu" "*.Mask") (remove_unused_layers no) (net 2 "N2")))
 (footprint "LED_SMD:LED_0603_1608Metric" (layer "F.Cu") (at 168.855 99.352)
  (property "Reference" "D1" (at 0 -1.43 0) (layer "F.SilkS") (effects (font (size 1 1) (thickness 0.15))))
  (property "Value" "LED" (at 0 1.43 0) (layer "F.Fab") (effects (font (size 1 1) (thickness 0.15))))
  (fp_line (start -1.485 -0.735) (end -1.485 0.735) (stroke (width 0.12) (type solid)) (layer "F.SilkS"))
  (fp_line (start -1.485 0.735) (end 0.8 0.735) (stroke (width 0.12) (type solid)) (layer "F.SilkS"))
  (fp_line (start 0.8 -0.735) (end -1.485 -0.735) (stroke (width 0.12) (type solid)) (layer "F.SilkS"))
  (pad "1" smd roundrect (at -0.7875 0) (size 0.875 0.95) (layers "F.Cu" "F.Paste" "F.Mask") (roundrect_rratio 0.25) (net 5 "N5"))
  (pad "2" smd roundrect (at 0.7875 0) (size 0.875 0.95) (layers "F.Cu" "F.Paste" "F.Mask") (roundrect_rratio 0.25) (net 1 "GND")))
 (gr_line (start 140 75) (end 140 105) (stroke (width 0.05) (type default)) (layer "Edge.Cuts"))
 (gr_arc (start 180 105) (mid 178.535534 108.535534) (end 175 110) (stroke (width 0.05) (type default)) (layer "Edge.Cuts"))
 (gr_line (start 145 110) (end 175 110) (stroke (width 0.05) (type default)) (layer "Edge.Cuts"))
 (gr_arc (start 175 70) (mid 178.535534 71.464466) (end 180 75) (stroke (width 0.05) (type default)) (layer "Edge.Cuts"))
 (gr_line (start 145 70) (end 175 70) (stroke (width 0.05) (type default)) (layer "Edge.Cuts"))
 (gr_arc (start 140 75) (mid 141.464466 71.464466) (end 145 70) (stroke (width 0.05) (type default)) (layer "Edge.Cuts"))
 (gr_arc (start 145 110) (mid 141.464466 108.535534) (end 140 105) (stroke (width 0.05) (type default)) (layer "Edge.Cuts"))
 (gr_line (start 180 105) (end 180 75) (stroke (width 0.05) (type default)) (layer "Edge.Cuts"))
 (segment (start 156.792 101.468) (end 156.792 89.932) (width 0.2) (layer "F.Cu") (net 2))
 (segment (start 156.792 89.932) (end 153.76 86.9) (width 0.2) (layer "F.Cu") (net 2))
 (segment (start 168.8425 100.127) (end 171.663 100.127) (width 0.2) (layer "F.Cu") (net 5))
 (segment (start 171.663 100.127) (end 172.43 99.36) (width 0.2) (layer "F.Cu") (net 5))
 (segment (start 168.0675 99.352) (end 168.8425 100.127) (width 0.2) (layer "F.Cu") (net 5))
 (segment (start 149.192 101.468) (end 150.292 102.568) (width 0.2) (layer "F.Cu") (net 3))
 (segment (start 150.292 102.568) (end 164.692 102.568) (width 0.2) (layer "F.Cu") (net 3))
 (segment (start 172.205 101.46) (end 173.7 99.965) (width 0.2) (layer "F.Cu") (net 3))
 (segment (start 173.7 99.965) (end 173.7 99.36) (width 0.2) (layer "F.Cu") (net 3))
 (segment (start 165.8 101.46) (end 172.205 101.46) (width 0.2) (layer "F.Cu") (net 3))
 (segment (start 164.692 102.568) (end 165.8 101.46) (width 0.2) (layer "F.Cu") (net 3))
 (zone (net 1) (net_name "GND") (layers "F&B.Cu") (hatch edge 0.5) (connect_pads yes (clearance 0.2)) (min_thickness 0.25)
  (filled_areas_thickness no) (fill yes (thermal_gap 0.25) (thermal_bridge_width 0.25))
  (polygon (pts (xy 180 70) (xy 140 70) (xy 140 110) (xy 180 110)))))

